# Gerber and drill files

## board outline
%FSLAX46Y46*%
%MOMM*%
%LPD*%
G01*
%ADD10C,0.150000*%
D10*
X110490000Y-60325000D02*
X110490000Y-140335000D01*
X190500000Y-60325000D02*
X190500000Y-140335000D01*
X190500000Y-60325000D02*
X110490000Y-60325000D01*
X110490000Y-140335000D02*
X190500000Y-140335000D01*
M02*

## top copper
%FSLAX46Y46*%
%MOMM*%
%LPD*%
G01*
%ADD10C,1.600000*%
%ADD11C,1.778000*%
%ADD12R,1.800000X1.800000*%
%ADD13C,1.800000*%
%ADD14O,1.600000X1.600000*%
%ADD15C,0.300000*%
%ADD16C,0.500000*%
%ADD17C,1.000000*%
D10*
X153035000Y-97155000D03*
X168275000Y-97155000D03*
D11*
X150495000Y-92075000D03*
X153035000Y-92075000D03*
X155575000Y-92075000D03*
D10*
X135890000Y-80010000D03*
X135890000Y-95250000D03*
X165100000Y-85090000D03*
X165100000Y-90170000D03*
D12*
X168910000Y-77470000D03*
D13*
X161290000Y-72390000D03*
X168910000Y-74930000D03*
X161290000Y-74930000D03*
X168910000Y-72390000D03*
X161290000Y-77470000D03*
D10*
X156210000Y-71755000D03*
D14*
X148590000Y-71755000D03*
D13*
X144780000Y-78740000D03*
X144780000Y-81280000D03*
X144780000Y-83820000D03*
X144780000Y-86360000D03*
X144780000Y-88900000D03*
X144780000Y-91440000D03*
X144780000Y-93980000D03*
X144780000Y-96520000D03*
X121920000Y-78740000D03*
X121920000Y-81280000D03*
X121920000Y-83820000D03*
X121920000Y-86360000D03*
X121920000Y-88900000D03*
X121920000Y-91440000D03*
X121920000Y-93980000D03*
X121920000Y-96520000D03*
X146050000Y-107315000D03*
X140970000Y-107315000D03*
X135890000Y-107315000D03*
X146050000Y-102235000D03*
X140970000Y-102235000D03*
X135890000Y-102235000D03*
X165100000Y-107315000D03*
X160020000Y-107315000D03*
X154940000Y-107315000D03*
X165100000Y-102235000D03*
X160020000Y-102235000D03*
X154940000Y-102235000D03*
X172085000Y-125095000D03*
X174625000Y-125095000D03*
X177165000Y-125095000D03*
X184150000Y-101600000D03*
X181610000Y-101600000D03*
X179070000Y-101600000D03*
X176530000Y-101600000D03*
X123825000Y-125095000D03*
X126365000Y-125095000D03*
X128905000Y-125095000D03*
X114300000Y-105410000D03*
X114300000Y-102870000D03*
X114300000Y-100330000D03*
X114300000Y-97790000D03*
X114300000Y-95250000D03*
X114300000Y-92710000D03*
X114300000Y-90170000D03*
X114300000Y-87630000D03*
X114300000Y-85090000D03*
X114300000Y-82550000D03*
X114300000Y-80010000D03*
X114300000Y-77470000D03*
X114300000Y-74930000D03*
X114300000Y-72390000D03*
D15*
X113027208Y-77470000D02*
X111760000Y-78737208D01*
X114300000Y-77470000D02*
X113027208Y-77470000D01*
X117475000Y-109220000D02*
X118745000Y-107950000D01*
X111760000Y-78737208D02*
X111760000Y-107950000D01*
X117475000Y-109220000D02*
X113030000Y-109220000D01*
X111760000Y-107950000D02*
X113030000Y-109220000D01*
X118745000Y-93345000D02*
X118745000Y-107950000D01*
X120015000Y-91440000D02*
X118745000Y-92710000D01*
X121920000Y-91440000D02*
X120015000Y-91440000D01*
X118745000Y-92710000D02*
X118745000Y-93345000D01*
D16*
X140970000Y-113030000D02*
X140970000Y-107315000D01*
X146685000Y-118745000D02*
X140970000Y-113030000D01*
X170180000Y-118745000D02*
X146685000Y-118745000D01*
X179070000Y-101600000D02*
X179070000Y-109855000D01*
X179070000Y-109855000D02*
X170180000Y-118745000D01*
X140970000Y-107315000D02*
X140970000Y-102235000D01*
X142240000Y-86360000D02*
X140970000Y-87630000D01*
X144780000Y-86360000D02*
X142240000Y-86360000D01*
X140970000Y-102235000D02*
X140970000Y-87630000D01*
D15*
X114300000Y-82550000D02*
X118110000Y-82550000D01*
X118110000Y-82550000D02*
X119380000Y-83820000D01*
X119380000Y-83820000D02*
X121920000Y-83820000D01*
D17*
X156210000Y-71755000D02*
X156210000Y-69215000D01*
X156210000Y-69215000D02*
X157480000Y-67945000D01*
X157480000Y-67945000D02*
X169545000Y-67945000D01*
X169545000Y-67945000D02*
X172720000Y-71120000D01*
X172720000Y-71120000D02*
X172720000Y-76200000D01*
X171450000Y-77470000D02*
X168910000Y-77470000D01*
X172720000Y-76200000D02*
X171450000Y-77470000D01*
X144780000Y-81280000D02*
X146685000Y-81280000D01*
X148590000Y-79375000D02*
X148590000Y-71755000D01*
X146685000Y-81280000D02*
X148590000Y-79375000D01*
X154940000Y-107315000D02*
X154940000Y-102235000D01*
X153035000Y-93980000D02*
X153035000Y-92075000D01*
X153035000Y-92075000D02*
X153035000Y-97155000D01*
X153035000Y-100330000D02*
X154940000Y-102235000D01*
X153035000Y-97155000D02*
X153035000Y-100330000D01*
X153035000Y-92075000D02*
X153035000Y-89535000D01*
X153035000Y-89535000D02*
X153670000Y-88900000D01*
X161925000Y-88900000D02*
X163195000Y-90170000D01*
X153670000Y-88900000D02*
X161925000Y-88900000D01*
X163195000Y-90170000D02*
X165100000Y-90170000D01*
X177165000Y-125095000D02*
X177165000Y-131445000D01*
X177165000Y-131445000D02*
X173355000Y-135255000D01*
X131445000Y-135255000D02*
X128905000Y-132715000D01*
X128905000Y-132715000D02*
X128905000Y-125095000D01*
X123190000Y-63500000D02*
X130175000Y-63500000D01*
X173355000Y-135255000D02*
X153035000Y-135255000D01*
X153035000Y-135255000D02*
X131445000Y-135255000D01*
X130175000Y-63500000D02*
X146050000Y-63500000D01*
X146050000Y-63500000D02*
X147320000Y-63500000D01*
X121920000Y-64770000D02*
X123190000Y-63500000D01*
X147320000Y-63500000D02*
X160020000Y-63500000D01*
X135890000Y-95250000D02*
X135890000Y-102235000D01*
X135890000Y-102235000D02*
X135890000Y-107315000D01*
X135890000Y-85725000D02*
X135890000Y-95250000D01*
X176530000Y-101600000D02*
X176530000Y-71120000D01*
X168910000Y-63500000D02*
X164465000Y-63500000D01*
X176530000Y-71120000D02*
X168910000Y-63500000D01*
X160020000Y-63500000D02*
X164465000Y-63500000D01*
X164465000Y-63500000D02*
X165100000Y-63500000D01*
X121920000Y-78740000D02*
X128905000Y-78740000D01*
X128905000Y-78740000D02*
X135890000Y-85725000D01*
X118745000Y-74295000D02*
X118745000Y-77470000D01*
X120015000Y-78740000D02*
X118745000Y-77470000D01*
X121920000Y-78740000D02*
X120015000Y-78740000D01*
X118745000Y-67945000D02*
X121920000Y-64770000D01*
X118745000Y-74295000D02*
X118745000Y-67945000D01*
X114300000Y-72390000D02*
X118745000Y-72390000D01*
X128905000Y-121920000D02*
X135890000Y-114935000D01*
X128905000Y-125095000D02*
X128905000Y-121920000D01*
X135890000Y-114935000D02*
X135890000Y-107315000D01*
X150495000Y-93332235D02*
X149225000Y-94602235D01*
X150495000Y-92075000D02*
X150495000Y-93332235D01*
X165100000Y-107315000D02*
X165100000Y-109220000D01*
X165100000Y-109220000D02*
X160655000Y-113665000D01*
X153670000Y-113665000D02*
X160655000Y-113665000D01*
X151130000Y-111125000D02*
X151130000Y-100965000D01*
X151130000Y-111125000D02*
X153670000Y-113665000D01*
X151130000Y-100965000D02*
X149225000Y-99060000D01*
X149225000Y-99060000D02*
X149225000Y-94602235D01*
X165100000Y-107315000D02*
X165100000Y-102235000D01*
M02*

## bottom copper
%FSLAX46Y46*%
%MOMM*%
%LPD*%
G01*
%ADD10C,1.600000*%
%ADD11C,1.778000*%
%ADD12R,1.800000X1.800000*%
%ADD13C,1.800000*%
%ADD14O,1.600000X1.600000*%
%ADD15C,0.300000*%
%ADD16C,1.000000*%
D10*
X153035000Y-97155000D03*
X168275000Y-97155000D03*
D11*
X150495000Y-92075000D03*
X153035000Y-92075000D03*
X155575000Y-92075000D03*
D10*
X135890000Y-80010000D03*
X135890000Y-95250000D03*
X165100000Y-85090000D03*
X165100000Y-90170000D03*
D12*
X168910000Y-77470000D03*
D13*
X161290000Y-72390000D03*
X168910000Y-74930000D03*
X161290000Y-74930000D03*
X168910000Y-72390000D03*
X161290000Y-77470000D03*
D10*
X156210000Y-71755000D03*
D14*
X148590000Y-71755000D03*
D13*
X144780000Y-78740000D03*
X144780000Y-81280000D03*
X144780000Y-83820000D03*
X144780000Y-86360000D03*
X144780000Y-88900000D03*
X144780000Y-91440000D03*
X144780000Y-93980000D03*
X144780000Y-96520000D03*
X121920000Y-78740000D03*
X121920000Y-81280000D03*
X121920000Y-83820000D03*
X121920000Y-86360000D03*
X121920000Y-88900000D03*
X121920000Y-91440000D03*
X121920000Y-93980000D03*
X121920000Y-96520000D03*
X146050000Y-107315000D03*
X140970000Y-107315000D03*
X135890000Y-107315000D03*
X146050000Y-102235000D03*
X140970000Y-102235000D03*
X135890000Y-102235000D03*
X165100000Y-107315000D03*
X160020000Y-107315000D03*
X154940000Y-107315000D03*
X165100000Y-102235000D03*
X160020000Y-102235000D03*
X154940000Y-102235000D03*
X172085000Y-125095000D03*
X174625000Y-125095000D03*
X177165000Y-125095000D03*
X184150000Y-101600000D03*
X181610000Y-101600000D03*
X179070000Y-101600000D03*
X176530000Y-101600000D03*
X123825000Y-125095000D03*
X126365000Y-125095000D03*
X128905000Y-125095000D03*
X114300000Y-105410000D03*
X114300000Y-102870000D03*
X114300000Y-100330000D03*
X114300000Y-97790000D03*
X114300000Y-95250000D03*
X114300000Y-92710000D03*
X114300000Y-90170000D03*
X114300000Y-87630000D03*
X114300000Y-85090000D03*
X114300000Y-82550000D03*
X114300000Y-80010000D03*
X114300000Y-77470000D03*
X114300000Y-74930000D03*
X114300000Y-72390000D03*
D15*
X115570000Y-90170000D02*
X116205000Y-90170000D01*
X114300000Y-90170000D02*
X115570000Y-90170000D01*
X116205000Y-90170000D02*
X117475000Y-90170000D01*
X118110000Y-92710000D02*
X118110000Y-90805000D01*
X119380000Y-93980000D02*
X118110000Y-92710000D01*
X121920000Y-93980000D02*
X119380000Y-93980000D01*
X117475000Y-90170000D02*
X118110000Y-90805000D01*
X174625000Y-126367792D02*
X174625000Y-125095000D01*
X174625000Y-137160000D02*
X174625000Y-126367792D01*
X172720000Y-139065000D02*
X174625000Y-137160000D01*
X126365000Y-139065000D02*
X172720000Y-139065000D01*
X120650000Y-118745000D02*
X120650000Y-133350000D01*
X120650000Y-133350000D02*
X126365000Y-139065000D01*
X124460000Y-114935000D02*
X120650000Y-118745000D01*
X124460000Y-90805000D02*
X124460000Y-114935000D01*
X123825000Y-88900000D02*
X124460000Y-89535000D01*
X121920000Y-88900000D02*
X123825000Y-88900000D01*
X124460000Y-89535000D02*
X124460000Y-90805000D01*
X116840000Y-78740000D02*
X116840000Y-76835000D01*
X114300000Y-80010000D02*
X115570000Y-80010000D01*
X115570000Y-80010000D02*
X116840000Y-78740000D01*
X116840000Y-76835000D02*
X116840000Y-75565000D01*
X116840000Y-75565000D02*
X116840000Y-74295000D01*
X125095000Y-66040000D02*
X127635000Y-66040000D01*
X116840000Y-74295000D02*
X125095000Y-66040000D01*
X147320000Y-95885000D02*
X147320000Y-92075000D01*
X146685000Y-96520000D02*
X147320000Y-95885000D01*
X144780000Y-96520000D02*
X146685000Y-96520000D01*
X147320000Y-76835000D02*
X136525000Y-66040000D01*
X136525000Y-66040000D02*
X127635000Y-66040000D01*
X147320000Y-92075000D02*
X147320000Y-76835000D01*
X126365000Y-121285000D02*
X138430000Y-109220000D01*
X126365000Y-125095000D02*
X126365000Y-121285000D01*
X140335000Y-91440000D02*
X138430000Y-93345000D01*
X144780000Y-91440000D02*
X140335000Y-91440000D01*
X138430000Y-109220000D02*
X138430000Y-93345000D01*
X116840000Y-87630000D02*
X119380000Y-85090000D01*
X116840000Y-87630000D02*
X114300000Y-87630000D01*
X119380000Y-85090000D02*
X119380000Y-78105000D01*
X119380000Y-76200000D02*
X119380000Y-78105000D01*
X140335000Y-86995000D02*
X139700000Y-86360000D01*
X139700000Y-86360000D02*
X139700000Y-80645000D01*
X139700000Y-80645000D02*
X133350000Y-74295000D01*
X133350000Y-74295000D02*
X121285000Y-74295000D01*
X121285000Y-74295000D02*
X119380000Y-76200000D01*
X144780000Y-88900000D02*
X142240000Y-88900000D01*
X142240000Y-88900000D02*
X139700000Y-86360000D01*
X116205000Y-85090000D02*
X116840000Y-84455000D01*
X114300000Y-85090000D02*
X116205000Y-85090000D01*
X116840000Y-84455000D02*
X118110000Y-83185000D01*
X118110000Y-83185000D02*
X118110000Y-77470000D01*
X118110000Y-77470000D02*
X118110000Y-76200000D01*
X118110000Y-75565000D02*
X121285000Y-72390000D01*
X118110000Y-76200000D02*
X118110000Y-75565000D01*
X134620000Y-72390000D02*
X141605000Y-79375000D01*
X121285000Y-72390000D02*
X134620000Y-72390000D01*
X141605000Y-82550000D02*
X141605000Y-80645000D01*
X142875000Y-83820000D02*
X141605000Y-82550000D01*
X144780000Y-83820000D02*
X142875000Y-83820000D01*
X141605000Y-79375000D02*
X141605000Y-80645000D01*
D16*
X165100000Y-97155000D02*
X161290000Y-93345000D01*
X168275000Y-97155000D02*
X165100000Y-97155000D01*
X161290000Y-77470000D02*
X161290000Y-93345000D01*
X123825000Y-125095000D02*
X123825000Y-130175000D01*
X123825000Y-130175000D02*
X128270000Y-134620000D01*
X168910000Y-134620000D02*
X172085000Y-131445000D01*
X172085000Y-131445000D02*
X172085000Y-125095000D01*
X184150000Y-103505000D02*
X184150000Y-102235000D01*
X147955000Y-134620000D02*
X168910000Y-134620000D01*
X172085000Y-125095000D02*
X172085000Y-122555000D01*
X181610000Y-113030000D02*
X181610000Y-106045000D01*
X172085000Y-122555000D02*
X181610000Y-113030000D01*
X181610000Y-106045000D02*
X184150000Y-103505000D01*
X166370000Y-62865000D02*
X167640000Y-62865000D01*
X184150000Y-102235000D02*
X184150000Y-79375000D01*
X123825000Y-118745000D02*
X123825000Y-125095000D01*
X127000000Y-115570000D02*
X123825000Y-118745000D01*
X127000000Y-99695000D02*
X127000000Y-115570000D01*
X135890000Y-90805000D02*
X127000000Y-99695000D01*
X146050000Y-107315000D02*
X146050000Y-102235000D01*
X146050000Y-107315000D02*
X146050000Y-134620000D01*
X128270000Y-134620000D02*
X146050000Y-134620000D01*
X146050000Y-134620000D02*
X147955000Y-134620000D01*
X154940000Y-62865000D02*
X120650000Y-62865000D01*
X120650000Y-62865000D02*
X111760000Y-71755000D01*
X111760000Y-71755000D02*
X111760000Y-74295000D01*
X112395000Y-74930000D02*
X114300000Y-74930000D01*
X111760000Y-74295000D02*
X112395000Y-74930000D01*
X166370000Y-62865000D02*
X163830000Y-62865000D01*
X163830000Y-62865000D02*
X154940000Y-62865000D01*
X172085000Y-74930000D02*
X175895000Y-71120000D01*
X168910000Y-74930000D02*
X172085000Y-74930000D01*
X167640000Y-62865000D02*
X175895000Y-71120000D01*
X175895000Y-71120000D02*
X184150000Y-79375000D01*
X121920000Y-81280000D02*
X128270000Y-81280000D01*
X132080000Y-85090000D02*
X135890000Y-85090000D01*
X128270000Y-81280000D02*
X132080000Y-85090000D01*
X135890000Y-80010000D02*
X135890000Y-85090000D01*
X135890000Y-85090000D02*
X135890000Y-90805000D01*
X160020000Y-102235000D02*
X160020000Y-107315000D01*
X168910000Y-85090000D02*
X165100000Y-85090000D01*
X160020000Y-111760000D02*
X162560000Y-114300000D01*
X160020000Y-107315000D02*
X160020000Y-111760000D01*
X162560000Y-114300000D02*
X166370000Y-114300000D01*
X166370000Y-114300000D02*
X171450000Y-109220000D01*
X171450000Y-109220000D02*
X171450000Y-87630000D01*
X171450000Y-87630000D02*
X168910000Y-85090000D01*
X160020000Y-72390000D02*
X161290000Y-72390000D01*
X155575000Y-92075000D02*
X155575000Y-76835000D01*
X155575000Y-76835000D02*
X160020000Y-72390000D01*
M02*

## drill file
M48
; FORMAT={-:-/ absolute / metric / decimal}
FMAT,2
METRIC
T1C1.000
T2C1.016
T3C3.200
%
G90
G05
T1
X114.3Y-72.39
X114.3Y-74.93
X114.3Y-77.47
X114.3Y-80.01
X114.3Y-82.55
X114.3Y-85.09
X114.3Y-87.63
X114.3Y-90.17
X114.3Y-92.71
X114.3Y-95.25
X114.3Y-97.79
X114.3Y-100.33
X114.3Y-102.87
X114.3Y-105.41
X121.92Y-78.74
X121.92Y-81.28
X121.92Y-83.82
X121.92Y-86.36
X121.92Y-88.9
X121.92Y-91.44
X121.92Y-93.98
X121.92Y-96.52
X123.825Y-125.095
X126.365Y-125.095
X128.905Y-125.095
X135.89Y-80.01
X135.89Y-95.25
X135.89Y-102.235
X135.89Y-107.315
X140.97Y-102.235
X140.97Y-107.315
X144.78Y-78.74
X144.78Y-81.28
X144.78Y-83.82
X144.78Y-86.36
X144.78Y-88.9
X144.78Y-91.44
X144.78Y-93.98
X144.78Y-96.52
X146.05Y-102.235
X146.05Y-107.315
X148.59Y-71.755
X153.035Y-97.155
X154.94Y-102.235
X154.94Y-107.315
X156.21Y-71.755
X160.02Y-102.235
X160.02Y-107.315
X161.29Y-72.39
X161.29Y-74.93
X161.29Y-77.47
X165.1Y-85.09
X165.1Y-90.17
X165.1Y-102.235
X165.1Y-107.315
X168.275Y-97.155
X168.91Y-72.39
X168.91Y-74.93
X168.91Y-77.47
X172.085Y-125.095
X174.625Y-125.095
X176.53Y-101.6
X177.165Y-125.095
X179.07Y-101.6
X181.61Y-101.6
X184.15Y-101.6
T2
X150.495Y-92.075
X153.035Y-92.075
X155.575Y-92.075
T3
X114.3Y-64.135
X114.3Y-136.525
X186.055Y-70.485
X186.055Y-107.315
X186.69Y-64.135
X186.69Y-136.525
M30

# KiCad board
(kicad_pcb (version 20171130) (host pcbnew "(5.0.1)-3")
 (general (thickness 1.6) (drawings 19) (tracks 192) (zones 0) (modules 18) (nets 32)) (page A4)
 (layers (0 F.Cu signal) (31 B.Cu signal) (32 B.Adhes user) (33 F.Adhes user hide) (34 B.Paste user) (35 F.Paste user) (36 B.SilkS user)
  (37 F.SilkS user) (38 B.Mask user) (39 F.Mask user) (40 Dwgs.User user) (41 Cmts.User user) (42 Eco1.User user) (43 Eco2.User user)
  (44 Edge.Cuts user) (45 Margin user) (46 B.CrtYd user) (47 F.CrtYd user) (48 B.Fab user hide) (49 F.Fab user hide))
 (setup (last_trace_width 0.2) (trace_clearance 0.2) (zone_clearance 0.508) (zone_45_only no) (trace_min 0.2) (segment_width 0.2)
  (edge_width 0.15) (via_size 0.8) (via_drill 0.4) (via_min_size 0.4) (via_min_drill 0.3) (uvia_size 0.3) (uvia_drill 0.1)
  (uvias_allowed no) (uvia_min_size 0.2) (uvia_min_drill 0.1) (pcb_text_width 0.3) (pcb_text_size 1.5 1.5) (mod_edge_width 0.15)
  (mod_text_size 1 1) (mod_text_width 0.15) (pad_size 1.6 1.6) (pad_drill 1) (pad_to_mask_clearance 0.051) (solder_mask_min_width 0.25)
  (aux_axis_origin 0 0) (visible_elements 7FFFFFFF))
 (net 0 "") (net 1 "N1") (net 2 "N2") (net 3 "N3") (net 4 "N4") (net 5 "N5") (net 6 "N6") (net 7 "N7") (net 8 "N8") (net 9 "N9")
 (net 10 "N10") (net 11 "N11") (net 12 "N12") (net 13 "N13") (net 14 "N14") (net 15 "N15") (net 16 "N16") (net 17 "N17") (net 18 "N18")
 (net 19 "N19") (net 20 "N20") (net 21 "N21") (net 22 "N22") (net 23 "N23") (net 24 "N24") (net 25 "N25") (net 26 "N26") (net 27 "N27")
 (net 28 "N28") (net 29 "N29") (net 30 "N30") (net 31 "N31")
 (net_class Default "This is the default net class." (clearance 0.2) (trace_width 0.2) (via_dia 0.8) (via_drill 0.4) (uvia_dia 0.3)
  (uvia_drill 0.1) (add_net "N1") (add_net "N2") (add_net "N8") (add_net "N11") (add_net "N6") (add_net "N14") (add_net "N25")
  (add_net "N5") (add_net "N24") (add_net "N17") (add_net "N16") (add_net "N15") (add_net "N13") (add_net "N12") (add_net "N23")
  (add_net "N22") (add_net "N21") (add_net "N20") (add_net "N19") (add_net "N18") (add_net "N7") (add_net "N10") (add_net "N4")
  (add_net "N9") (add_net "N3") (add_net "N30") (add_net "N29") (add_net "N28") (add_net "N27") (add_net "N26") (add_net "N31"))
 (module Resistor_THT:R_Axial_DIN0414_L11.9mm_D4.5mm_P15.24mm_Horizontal (layer F.Cu) (at 153.035 97.155)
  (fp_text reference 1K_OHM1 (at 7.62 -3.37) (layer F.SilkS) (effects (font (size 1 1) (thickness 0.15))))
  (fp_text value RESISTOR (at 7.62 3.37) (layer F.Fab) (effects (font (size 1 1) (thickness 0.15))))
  (pad 1 thru_hole circle (at 0 0) (size 1.6 1.6) (drill 1) (layers *.Cu *.Mask) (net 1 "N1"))
  (pad 2 thru_hole circle (at 15.24 0) (size 1.6 1.6) (drill 1) (layers *.Cu *.Mask) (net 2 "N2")))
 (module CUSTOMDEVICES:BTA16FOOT (layer F.Cu) (at 153.035 86.995)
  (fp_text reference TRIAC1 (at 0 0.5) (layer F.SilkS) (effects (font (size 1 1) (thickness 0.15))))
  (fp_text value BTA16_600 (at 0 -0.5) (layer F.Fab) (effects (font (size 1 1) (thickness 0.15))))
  (pad 1 thru_hole circle (at -2.54 5.08) (size 1.778 1.778) (drill 1.016) (layers *.Cu *.Mask) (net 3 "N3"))
  (pad 2 thru_hole circle (at 0 5.08) (size 1.778 1.778) (drill 1.016) (layers *.Cu *.Mask) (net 1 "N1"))
  (pad 3 thru_hole circle (at 2.54 5.08) (size 1.778 1.778) (drill 1.016) (layers *.Cu *.Mask) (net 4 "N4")))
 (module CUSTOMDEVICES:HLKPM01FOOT (layer B.Cu) (at 150.495 87.63 180)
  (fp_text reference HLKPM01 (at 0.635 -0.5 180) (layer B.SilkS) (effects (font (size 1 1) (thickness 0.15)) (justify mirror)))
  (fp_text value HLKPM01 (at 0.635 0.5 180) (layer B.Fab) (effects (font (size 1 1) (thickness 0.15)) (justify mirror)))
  (pad 3 thru_hole circle (at 14.605 7.62 180) (size 1.6 1.6) (drill 1) (layers *.Cu *.Mask) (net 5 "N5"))
  (pad 4 thru_hole circle (at 14.605 -7.62 180) (size 1.6 1.6) (drill 1) (layers *.Cu *.Mask) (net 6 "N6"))
  (pad 1 thru_hole circle (at -14.605 2.54 180) (size 1.6 1.6) (drill 1) (layers *.Cu *.Mask) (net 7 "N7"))
  (pad 2 thru_hole circle (at -14.605 -2.54 180) (size 1.6 1.6) (drill 1) (layers *.Cu *.Mask) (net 1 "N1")))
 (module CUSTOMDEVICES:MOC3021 (layer F.Cu) (at 168.91 77.47 180)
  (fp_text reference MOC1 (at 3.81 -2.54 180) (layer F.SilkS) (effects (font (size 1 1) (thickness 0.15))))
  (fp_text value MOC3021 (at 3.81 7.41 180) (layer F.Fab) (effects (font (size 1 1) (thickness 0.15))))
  (pad 1 thru_hole rect (at 0 0 180) (size 1.8 1.8) (drill 1) (layers *.Cu *.Mask) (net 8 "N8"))
  (pad 4 thru_hole circle (at 7.62 5.08 180) (size 1.8 1.8) (drill 1) (layers *.Cu *.Mask) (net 4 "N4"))
  (pad 2 thru_hole circle (at 0 2.54 180) (size 1.8 1.8) (drill 1) (layers *.Cu *.Mask) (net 5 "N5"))
  (pad 5 thru_hole circle (at 7.62 2.54 180) (size 1.8 1.8) (drill 1) (layers *.Cu *.Mask) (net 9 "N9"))
  (pad 3 thru_hole circle (at 0 5.08 180) (size 1.8 1.8) (drill 1) (layers *.Cu *.Mask) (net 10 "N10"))
  (pad 6 thru_hole circle (at 7.62 0 180) (size 1.8 1.8) (drill 1) (layers *.Cu *.Mask) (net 2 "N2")))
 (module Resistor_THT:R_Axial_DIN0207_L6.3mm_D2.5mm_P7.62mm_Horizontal (layer F.Cu) (at 156.21 71.755 180)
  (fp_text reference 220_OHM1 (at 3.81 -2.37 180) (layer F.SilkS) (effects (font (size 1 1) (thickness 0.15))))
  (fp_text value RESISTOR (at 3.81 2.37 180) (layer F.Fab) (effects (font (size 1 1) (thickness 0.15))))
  (pad 1 thru_hole circle (at 0 0 180) (size 1.6 1.6) (drill 1) (layers *.Cu *.Mask) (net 8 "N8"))
  (pad 2 thru_hole oval (at 7.62 0 180) (size 1.6 1.6) (drill 1) (layers *.Cu *.Mask) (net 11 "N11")))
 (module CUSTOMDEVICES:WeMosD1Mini (layer F.Cu) (at 133.35 86.36 180)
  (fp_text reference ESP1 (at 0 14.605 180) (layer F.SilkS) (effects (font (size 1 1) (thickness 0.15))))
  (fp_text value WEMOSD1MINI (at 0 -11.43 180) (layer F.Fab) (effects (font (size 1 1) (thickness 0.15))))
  (pad 16 thru_hole circle (at -11.43 7.62 180) (size 1.8 1.8) (drill 1) (layers *.Cu *.Mask) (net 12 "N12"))
  (pad 15 thru_hole circle (at -11.43 5.08 180) (size 1.8 1.8) (drill 1) (layers *.Cu *.Mask) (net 11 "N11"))
  (pad 14 thru_hole circle (at -11.43 2.54 180) (size 1.8 1.8) (drill 1) (layers *.Cu *.Mask) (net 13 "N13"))
  (pad 13 thru_hole circle (at -11.43 0 180) (size 1.8 1.8) (drill 1) (layers *.Cu *.Mask) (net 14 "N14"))
  (pad 12 thru_hole circle (at -11.43 -2.54 180) (size 1.8 1.8) (drill 1) (layers *.Cu *.Mask) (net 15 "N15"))
  (pad 11 thru_hole circle (at -11.43 -5.08 180) (size 1.8 1.8) (drill 1) (layers *.Cu *.Mask) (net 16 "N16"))
  (pad 10 thru_hole circle (at -11.43 -7.62 180) (size 1.8 1.8) (drill 1) (layers *.Cu *.Mask) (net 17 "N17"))
  (pad 9 thru_hole circle (at -11.43 -10.16 180) (size 1.8 1.8) (drill 1) (layers *.Cu *.Mask) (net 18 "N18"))
  (pad 8 thru_hole circle (at 11.43 7.62 180) (size 1.8 1.8) (drill 1) (layers *.Cu *.Mask) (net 6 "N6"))
  (pad 7 thru_hole circle (at 11.43 5.08 180) (size 1.8 1.8) (drill 1) (layers *.Cu *.Mask) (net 5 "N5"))
  (pad 6 thru_hole circle (at 11.43 2.54 180) (size 1.8 1.8) (drill 1) (layers *.Cu *.Mask) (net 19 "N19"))
  (pad 5 thru_hole circle (at 11.43 0 180) (size 1.8 1.8) (drill 1) (layers *.Cu *.Mask) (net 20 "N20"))
  (pad 4 thru_hole circle (at 11.43 -2.54 180) (size 1.8 1.8) (drill 1) (layers *.Cu *.Mask) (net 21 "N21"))
  (pad 3 thru_hole circle (at 11.43 -5.08 180) (size 1.8 1.8) (drill 1) (layers *.Cu *.Mask) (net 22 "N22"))
  (pad 2 thru_hole circle (at 11.43 -7.62 180) (size 1.8 1.8) (drill 1) (layers *.Cu *.Mask) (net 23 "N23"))
  (pad 1 thru_hole circle (at 11.43 -10.16 180) (size 1.8 1.8) (drill 1) (layers *.Cu *.Mask) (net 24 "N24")))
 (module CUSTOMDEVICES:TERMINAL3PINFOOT (layer B.Cu) (at 140.97 104.775)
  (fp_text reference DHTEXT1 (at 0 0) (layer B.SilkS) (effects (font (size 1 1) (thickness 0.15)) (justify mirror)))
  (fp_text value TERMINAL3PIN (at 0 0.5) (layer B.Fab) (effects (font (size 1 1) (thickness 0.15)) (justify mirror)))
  (pad 3 thru_hole circle (at 5.08 2.54) (size 1.8 1.8) (drill 1) (layers *.Cu *.Mask) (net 5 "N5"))
  (pad 2 thru_hole circle (at 0 2.54) (size 1.8 1.8) (drill 1) (layers *.Cu *.Mask) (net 14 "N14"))
  (pad 1 thru_hole circle (at -5.08 2.54) (size 1.8 1.8) (drill 1) (layers *.Cu *.Mask) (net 6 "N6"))
  (pad 3 thru_hole circle (at 5.08 -2.54) (size 1.8 1.8) (drill 1) (layers *.Cu *.Mask) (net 5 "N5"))
  (pad 2 thru_hole circle (at 0 -2.54) (size 1.8 1.8) (drill 1) (layers *.Cu *.Mask) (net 14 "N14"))
  (pad 1 thru_hole circle (at -5.08 -2.54) (size 1.8 1.8) (drill 1) (layers *.Cu *.Mask) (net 6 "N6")))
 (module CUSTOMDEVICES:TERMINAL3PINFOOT (layer B.Cu) (at 160.02 104.775)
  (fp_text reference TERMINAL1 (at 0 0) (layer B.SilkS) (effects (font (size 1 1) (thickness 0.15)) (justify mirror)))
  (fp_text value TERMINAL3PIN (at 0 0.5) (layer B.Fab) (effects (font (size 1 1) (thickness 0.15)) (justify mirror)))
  (pad 3 thru_hole circle (at 5.08 2.54) (size 1.8 1.8) (drill 1) (layers *.Cu *.Mask) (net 3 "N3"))
  (pad 2 thru_hole circle (at 0 2.54) (size 1.8 1.8) (drill 1) (layers *.Cu *.Mask) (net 7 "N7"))
  (pad 1 thru_hole circle (at -5.08 2.54) (size 1.8 1.8) (drill 1) (layers *.Cu *.Mask) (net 1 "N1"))
  (pad 3 thru_hole circle (at 5.08 -2.54) (size 1.8 1.8) (drill 1) (layers *.Cu *.Mask) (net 3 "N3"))
  (pad 2 thru_hole circle (at 0 -2.54) (size 1.8 1.8) (drill 1) (layers *.Cu *.Mask) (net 7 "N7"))
  (pad 1 thru_hole circle (at -5.08 -2.54) (size 1.8 1.8) (drill 1) (layers *.Cu *.Mask) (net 1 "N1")))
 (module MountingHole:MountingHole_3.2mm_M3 (layer F.Cu) (at 186.055 107.315)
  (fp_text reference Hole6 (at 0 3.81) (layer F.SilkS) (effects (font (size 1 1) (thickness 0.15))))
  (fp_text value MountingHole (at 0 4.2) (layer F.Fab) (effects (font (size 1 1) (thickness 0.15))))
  (pad 1 np_thru_hole circle (at 0 0) (size 3.2 3.2) (drill 3.2) (layers *.Cu *.Mask)))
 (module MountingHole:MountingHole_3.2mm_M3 (layer F.Cu) (at 186.055 70.485)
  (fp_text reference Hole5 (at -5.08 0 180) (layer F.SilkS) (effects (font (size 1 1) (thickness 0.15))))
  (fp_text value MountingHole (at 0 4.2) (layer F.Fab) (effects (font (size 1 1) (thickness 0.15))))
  (pad 1 np_thru_hole circle (at 0 0) (size 3.2 3.2) (drill 3.2) (layers *.Cu *.Mask)))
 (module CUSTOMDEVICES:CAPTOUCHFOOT (layer F.Cu) (at 174.625 130.175 180)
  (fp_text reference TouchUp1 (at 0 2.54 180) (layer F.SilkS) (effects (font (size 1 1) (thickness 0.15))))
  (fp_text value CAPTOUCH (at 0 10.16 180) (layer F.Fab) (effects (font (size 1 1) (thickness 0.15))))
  (pad 3 thru_hole circle (at 2.54 5.08 180) (size 1.8 1.8) (drill 1) (layers *.Cu *.Mask) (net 5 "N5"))
  (pad 2 thru_hole circle (at 0 5.08 180) (size 1.8 1.8) (drill 1) (layers *.Cu *.Mask) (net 21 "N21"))
  (pad 1 thru_hole circle (at -2.54 5.08 180) (size 1.8 1.8) (drill 1) (layers *.Cu *.Mask) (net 6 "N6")))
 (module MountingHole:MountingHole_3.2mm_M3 (layer F.Cu) (at 186.69 136.525)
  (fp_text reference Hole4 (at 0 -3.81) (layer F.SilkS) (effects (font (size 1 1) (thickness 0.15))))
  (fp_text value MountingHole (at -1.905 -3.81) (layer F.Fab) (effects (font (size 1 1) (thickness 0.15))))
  (pad 1 np_thru_hole circle (at 0 0) (size 3.2 3.2) (drill 3.2) (layers *.Cu *.Mask)))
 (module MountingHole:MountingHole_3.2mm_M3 (layer F.Cu) (at 114.3 136.525)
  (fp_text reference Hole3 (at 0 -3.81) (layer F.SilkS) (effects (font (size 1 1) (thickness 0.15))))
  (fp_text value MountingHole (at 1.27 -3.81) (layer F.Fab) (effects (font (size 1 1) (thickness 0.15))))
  (pad 1 np_thru_hole circle (at 0 0) (size 3.2 3.2) (drill 3.2) (layers *.Cu *.Mask)))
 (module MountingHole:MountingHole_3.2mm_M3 (layer F.Cu) (at 186.69 64.135)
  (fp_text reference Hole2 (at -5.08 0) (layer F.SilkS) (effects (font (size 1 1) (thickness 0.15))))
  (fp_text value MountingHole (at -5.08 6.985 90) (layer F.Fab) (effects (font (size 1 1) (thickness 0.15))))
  (pad 1 np_thru_hole circle (at 0 0) (size 3.2 3.2) (drill 3.2) (layers *.Cu *.Mask)))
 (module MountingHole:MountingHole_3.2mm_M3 (layer F.Cu) (at 114.3 64.135)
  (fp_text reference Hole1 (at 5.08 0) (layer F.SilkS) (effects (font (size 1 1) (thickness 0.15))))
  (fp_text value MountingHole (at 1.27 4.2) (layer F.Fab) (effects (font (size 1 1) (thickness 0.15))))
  (pad 1 np_thru_hole circle (at 0 0) (size 3.2 3.2) (drill 3.2) (layers *.Cu *.Mask)))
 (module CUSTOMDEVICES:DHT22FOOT (layer F.Cu) (at 181.61 88.9)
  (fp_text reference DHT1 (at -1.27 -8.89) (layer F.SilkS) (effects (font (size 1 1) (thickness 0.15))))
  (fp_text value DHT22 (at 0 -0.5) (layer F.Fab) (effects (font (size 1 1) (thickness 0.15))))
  (pad 4 thru_hole circle (at 2.54 12.7) (size 1.8 1.8) (drill 1) (layers *.Cu *.Mask) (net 5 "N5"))
  (pad 3 thru_hole circle (at 0 12.7) (size 1.8 1.8) (drill 1) (layers *.Cu *.Mask) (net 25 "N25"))
  (pad 2 thru_hole circle (at -2.54 12.7) (size 1.8 1.8) (drill 1) (layers *.Cu *.Mask) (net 14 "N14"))
  (pad 1 thru_hole circle (at -5.08 12.7) (size 1.8 1.8) (drill 1) (layers *.Cu *.Mask) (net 6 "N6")))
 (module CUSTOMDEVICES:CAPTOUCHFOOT (layer F.Cu) (at 126.365 130.175 180)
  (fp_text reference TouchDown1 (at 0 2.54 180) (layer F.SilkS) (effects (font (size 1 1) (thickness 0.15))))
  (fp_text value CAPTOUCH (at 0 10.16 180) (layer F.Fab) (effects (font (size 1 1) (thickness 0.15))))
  (pad 3 thru_hole circle (at 2.54 5.08 180) (size 1.8 1.8) (drill 1) (layers *.Cu *.Mask) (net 5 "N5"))
  (pad 2 thru_hole circle (at 0 5.08 180) (size 1.8 1.8) (drill 1) (layers *.Cu *.Mask) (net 16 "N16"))
  (pad 1 thru_hole circle (at -2.54 5.08 180) (size 1.8 1.8) (drill 1) (layers *.Cu *.Mask) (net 6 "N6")))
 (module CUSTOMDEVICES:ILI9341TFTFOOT (layer F.Cu) (at 116.84 90.17 180)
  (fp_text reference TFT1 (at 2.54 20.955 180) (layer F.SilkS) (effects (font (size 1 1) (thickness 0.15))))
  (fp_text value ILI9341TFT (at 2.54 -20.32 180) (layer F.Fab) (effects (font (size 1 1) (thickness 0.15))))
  (pad 14 thru_hole circle (at 2.54 -15.24 180) (size 1.8 1.8) (drill 1) (layers *.Cu *.Mask) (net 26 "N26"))
  (pad 13 thru_hole circle (at 2.54 -12.7 180) (size 1.8 1.8) (drill 1) (layers *.Cu *.Mask) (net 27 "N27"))
  (pad 12 thru_hole circle (at 2.54 -10.16 180) (size 1.8 1.8) (drill 1) (layers *.Cu *.Mask) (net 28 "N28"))
  (pad 11 thru_hole circle (at 2.54 -7.62 180) (size 1.8 1.8) (drill 1) (layers *.Cu *.Mask) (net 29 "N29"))
  (pad 10 thru_hole circle (at 2.54 -5.08 180) (size 1.8 1.8) (drill 1) (layers *.Cu *.Mask) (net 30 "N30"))
  (pad 9 thru_hole circle (at 2.54 -2.54 180) (size 1.8 1.8) (drill 1) (layers *.Cu *.Mask) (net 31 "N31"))
  (pad 8 thru_hole circle (at 2.54 0 180) (size 1.8 1.8) (drill 1) (layers *.Cu *.Mask) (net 23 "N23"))
  (pad 7 thru_hole circle (at 2.54 2.54 180) (size 1.8 1.8) (drill 1) (layers *.Cu *.Mask) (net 15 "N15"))
  (pad 6 thru_hole circle (at 2.54 5.08 180) (size 1.8 1.8) (drill 1) (layers *.Cu *.Mask) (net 13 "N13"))
  (pad 5 thru_hole circle (at 2.54 7.62 180) (size 1.8 1.8) (drill 1) (layers *.Cu *.Mask) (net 19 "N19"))
  (pad 4 thru_hole circle (at 2.54 10.16 180) (size 1.8 1.8) (drill 1) (layers *.Cu *.Mask) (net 18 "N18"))
  (pad 3 thru_hole circle (at 2.54 12.7 180) (size 1.8 1.8) (drill 1) (layers *.Cu *.Mask) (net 22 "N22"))
  (pad 2 thru_hole circle (at 2.54 15.24 180) (size 1.8 1.8) (drill 1) (layers *.Cu *.Mask) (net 5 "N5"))
  (pad 1 thru_hole circle (at 2.54 17.78 180) (size 1.8 1.8) (drill 1) (layers *.Cu *.Mask) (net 6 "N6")))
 (gr_line (start 110.49 60.325) (end 110.49 140.335) (layer Edge.Cuts) (width 0.15))
 (gr_line (start 190.5 60.325) (end 190.5 140.335) (layer Edge.Cuts) (width 0.15))
 (gr_line (start 190.5 60.325) (end 110.49 60.325) (layer Edge.Cuts) (width 0.15))
 (gr_line (start 110.49 140.335) (end 190.5 140.335) (layer Edge.Cuts) (width 0.15))
 (segment (start 115.57 90.17) (end 116.205 90.17) (width 0.3) (layer B.Cu) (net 23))
 (segment (start 114.3 90.17) (end 115.57 90.17) (width 0.3) (layer B.Cu) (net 23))
 (segment (start 116.205 90.17) (end 117.475 90.17) (width 0.3) (layer B.Cu) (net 23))
 (segment (start 118.11 92.71) (end 118.11 90.805) (width 0.3) (layer B.Cu) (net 23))
 (segment (start 119.38 93.98) (end 118.11 92.71) (width 0.3) (layer B.Cu) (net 23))
 (segment (start 121.92 93.98) (end 119.38 93.98) (width 0.3) (layer B.Cu) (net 23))
 (segment (start 117.475 90.17) (end 118.11 90.805) (width 0.3) (layer B.Cu) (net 23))
 (segment (start 113.027208 77.47) (end 111.76 78.737208) (width 0.3) (layer F.Cu) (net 22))
 (segment (start 114.3 77.47) (end 113.027208 77.47) (width 0.3) (layer F.Cu) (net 22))
 (segment (start 117.475 109.22) (end 118.745 107.95) (width 0.3) (layer F.Cu) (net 22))
 (segment (start 111.76 78.737208) (end 111.76 107.95) (width 0.3) (layer F.Cu) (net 22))
 (segment (start 117.475 109.22) (end 113.03 109.22) (width 0.3) (layer F.Cu) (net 22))
 (segment (start 111.76 107.95) (end 113.03 109.22) (width 0.3) (layer F.Cu) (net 22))
 (segment (start 118.745 93.345) (end 118.745 107.95) (width 0.3) (layer F.Cu) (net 22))
 (segment (start 120.015 91.44) (end 118.745 92.71) (width 0.3) (layer F.Cu) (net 22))
 (segment (start 121.92 91.44) (end 120.015 91.44) (width 0.3) (layer F.Cu) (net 22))
 (segment (start 118.745 92.71) (end 118.745 93.345) (width 0.3) (layer F.Cu) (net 22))
 (segment (start 174.625 126.367792) (end 174.625 125.095) (width 0.3) (layer B.Cu) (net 21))
 (segment (start 174.625 137.16) (end 174.625 126.367792) (width 0.3) (layer B.Cu) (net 21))
 (segment (start 172.72 139.065) (end 174.625 137.16) (width 0.3) (layer B.Cu) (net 21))
 (segment (start 126.365 139.065) (end 172.72 139.065) (width 0.3) (layer B.Cu) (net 21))
 (segment (start 120.65 118.745) (end 120.65 133.35) (width 0.3) (layer B.Cu) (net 21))
 (segment (start 120.65 133.35) (end 126.365 139.065) (width 0.3) (layer B.Cu) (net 21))
 (segment (start 124.46 114.935) (end 120.65 118.745) (width 0.3) (layer B.Cu) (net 21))
 (segment (start 124.46 90.805) (end 124.46 114.935) (width 0.3) (layer B.Cu) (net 21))
 (segment (start 123.825 88.9) (end 124.46 89.535) (width 0.3) (layer B.Cu) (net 21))
 (segment (start 121.92 88.9) (end 123.825 88.9) (width 0.3) (layer B.Cu) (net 21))
 (segment (start 124.46 89.535) (end 124.46 90.805) (width 0.3) (layer B.Cu) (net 21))
 (segment (start 140.97 113.03) (end 140.97 107.315) (width 0.5) (layer F.Cu) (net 14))
 (segment (start 146.685 118.745) (end 140.97 113.03) (width 0.5) (layer F.Cu) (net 14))
 (segment (start 170.18 118.745) (end 146.685 118.745) (width 0.5) (layer F.Cu) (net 14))
 (segment (start 179.07 101.6) (end 179.07 109.855) (width 0.5) (layer F.Cu) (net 14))
 (segment (start 179.07 109.855) (end 170.18 118.745) (width 0.5) (layer F.Cu) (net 14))
 (segment (start 140.97 107.315) (end 140.97 102.235) (width 0.5) (layer F.Cu) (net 14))
 (segment (start 142.24 86.36) (end 140.97 87.63) (width 0.5) (layer F.Cu) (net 14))
 (segment (start 144.78 86.36) (end 142.24 86.36) (width 0.5) (layer F.Cu) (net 14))
 (segment (start 140.97 102.235) (end 140.97 87.63) (width 0.5) (layer F.Cu) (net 14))
 (segment (start 114.3 82.55) (end 118.11 82.55) (width 0.3) (layer F.Cu) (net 19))
 (segment (start 118.11 82.55) (end 119.38 83.82) (width 0.3) (layer F.Cu) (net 19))
 (segment (start 119.38 83.82) (end 121.92 83.82) (width 0.3) (layer F.Cu) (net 19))
 (segment (start 116.84 78.74) (end 116.84 76.835) (width 0.3) (layer B.Cu) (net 18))
 (segment (start 114.3 80.01) (end 115.57 80.01) (width 0.3) (layer B.Cu) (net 18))
 (segment (start 115.57 80.01) (end 116.84 78.74) (width 0.3) (layer B.Cu) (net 18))
 (segment (start 116.84 76.835) (end 116.84 75.565) (width 0.3) (layer B.Cu) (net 18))
 (segment (start 116.84 75.565) (end 116.84 74.295) (width 0.3) (layer B.Cu) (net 18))
 (segment (start 125.095 66.04) (end 127.635 66.04) (width 0.3) (layer B.Cu) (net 18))
 (segment (start 116.84 74.295) (end 125.095 66.04) (width 0.3) (layer B.Cu) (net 18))
 (segment (start 147.32 95.885) (end 147.32 92.075) (width 0.3) (layer B.Cu) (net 18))
 (segment (start 146.685 96.52) (end 147.32 95.885) (width 0.3) (layer B.Cu) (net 18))
 (segment (start 144.78 96.52) (end 146.685 96.52) (width 0.3) (layer B.Cu) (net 18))
 (segment (start 147.32 76.835) (end 136.525 66.04) (width 0.3) (layer B.Cu) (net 18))
 (segment (start 136.525 66.04) (end 127.635 66.04) (width 0.3) (layer B.Cu) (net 18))
 (segment (start 147.32 92.075) (end 147.32 76.835) (width 0.3) (layer B.Cu) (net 18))
 (segment (start 126.365 121.285) (end 138.43 109.22) (width 0.3) (layer B.Cu) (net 16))
 (segment (start 126.365 125.095) (end 126.365 121.285) (width 0.3) (layer B.Cu) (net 16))
 (segment (start 140.335 91.44) (end 138.43 93.345) (width 0.3) (layer B.Cu) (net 16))
 (segment (start 144.78 91.44) (end 140.335 91.44) (width 0.3) (layer B.Cu) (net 16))
 (segment (start 138.43 109.22) (end 138.43 93.345) (width 0.3) (layer B.Cu) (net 16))
 (segment (start 116.84 87.63) (end 119.38 85.09) (width 0.3) (layer B.Cu) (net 15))
 (segment (start 116.84 87.63) (end 114.3 87.63) (width 0.3) (layer B.Cu) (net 15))
 (segment (start 119.38 85.09) (end 119.38 78.105) (width 0.3) (layer B.Cu) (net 15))
 (segment (start 119.38 76.2) (end 119.38 78.105) (width 0.3) (layer B.Cu) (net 15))
 (segment (start 140.335 86.995) (end 139.7 86.36) (width 0.3) (layer B.Cu) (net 15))
 (segment (start 139.7 86.36) (end 139.7 80.645) (width 0.3) (layer B.Cu) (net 15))
 (segment (start 139.7 80.645) (end 133.35 74.295) (width 0.3) (layer B.Cu) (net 15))
 (segment (start 133.35 74.295) (end 121.285 74.295) (width 0.3) (layer B.Cu) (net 15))
 (segment (start 121.285 74.295) (end 119.38 76.2) (width 0.3) (layer B.Cu) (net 15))
 (segment (start 144.78 88.9) (end 142.24 88.9) (width 0.3) (layer B.Cu) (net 15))
 (segment (start 142.24 88.9) (end 139.7 86.36) (width 0.3) (layer B.Cu) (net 15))
 (segment (start 116.205 85.09) (end 116.84 84.455) (width 0.3) (layer B.Cu) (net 13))
 (segment (start 114.3 85.09) (end 116.205 85.09) (width 0.3) (layer B.Cu) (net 13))
 (segment (start 116.84 84.455) (end 118.11 83.185) (width 0.3) (layer B.Cu) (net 13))
 (segment (start 118.11 83.185) (end 118.11 77.47) (width 0.3) (layer B.Cu) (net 13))
 (segment (start 118.11 77.47) (end 118.11 76.2) (width 0.3) (layer B.Cu) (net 13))
 (segment (start 118.11 75.565) (end 121.285 72.39) (width 0.3) (layer B.Cu) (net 13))
 (segment (start 118.11 76.2) (end 118.11 75.565) (width 0.3) (layer B.Cu) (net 13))
 (segment (start 134.62 72.39) (end 141.605 79.375) (width 0.3) (layer B.Cu) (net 13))
 (segment (start 121.285 72.39) (end 134.62 72.39) (width 0.3) (layer B.Cu) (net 13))
 (segment (start 141.605 82.55) (end 141.605 80.645) (width 0.3) (layer B.Cu) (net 13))
 (segment (start 142.875 83.82) (end 141.605 82.55) (width 0.3) (layer B.Cu) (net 13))
 (segment (start 144.78 83.82) (end 142.875 83.82) (width 0.3) (layer B.Cu) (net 13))
 (segment (start 141.605 79.375) (end 141.605 80.645) (width 0.3) (layer B.Cu) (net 13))
 (segment (start 156.21 71.755) (end 156.21 69.215) (width 1) (layer F.Cu) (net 8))
 (segment (start 156.21 69.215) (end 157.48 67.945) (width 1) (layer F.Cu) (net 8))
 (segment (start 157.48 67.945) (end 169.545 67.945) (width 1) (layer F.Cu) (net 8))
 (segment (start 169.545 67.945) (end 172.72 71.12) (width 1) (layer F.Cu) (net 8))
 (segment (start 172.72 71.12) (end 172.72 76.2) (width 1) (layer F.Cu) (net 8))
 (segment (start 171.45 77.47) (end 168.91 77.47) (width 1) (layer F.Cu) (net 8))
 (segment (start 172.72 76.2) (end 171.45 77.47) (width 1) (layer F.Cu) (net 8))
 (segment (start 144.78 81.28) (end 146.685 81.28) (width 1) (layer F.Cu) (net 11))
 (segment (start 148.59 79.375) (end 148.59 71.755) (width 1) (layer F.Cu) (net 11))
 (segment (start 146.685 81.28) (end 148.59 79.375) (width 1) (layer F.Cu) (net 11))
 (segment (start 165.1 97.155) (end 161.29 93.345) (width 1) (layer B.Cu) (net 2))
 (segment (start 168.275 97.155) (end 165.1 97.155) (width 1) (layer B.Cu) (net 2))
 (segment (start 161.29 77.47) (end 161.29 93.345) (width 1) (layer B.Cu) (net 2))
 (segment (start 154.94 107.315) (end 154.94 102.235) (width 1) (layer F.Cu) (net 1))
 (segment (start 153.035 93.98) (end 153.035 92.075) (width 1) (layer F.Cu) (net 1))
 (segment (start 153.035 92.075) (end 153.035 97.155) (width 1) (layer F.Cu) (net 1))
 (segment (start 153.035 100.33) (end 154.94 102.235) (width 1) (layer F.Cu) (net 1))
 (segment (start 153.035 97.155) (end 153.035 100.33) (width 1) (layer F.Cu) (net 1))
 (segment (start 153.035 92.075) (end 153.035 89.535) (width 1) (layer F.Cu) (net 1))
 (segment (start 153.035 89.535) (end 153.67 88.9) (width 1) (layer F.Cu) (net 1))
 (segment (start 161.925 88.9) (end 163.195 90.17) (width 1) (layer F.Cu) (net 1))
 (segment (start 153.67 88.9) (end 161.925 88.9) (width 1) (layer F.Cu) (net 1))
 (segment (start 163.195 90.17) (end 165.1 90.17) (width 1) (layer F.Cu) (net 1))
 (segment (start 177.165 125.095) (end 177.165 131.445) (width 1) (layer F.Cu) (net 6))
 (segment (start 177.165 131.445) (end 173.355 135.255) (width 1) (layer F.Cu) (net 6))
 (segment (start 131.445 135.255) (end 128.905 132.715) (width 1) (layer F.Cu) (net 6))
 (segment (start 128.905 132.715) (end 128.905 125.095) (width 1) (layer F.Cu) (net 6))
 (segment (start 123.19 63.5) (end 130.175 63.5) (width 1) (layer F.Cu) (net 6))
 (segment (start 173.355 135.255) (end 153.035 135.255) (width 1) (layer F.Cu) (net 6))
 (segment (start 153.035 135.255) (end 131.445 135.255) (width 1) (layer F.Cu) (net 6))
 (segment (start 130.175 63.5) (end 146.05 63.5) (width 1) (layer F.Cu) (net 6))
 (segment (start 146.05 63.5) (end 147.32 63.5) (width 1) (layer F.Cu) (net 6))
 (segment (start 121.92 64.77) (end 123.19 63.5) (width 1) (layer F.Cu) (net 6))
 (segment (start 147.32 63.5) (end 160.02 63.5) (width 1) (layer F.Cu) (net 6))
 (segment (start 135.89 95.25) (end 135.89 102.235) (width 1) (layer F.Cu) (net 6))
 (segment (start 135.89 102.235) (end 135.89 107.315) (width 1) (layer F.Cu) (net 6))
 (segment (start 135.89 85.725) (end 135.89 95.25) (width 1) (layer F.Cu) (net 6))
 (segment (start 176.53 101.6) (end 176.53 71.12) (width 1) (layer F.Cu) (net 6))
 (segment (start 168.91 63.5) (end 164.465 63.5) (width 1) (layer F.Cu) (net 6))
 (segment (start 176.53 71.12) (end 168.91 63.5) (width 1) (layer F.Cu) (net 6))
 (segment (start 160.02 63.5) (end 164.465 63.5) (width 1) (layer F.Cu) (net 6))
 (segment (start 164.465 63.5) (end 165.1 63.5) (width 1) (layer F.Cu) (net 6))
 (segment (start 121.92 78.74) (end 128.905 78.74) (width 1) (layer F.Cu) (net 6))
 (segment (start 128.905 78.74) (end 135.89 85.725) (width 1) (layer F.Cu) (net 6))
 (segment (start 118.745 74.295) (end 118.745 77.47) (width 1) (layer F.Cu) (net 6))
 (segment (start 120.015 78.74) (end 118.745 77.47) (width 1) (layer F.Cu) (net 6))
 (segment (start 121.92 78.74) (end 120.015 78.74) (width 1) (layer F.Cu) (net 6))
 (segment (start 118.745 67.945) (end 121.92 64.77) (width 1) (layer F.Cu) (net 6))
 (segment (start 118.745 74.295) (end 118.745 67.945) (width 1) (layer F.Cu) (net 6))
 (segment (start 114.3 72.39) (end 118.745 72.39) (width 1) (layer F.Cu) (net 6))
 (segment (start 128.905 121.92) (end 135.89 114.935) (width 1) (layer F.Cu) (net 6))
 (segment (start 128.905 125.095) (end 128.905 121.92) (width 1) (layer F.Cu) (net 6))
 (segment (start 135.89 114.935) (end 135.89 107.315) (width 1) (layer F.Cu) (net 6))
 (segment (start 123.825 125.095) (end 123.825 130.175) (width 1) (layer B.Cu) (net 5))
 (segment (start 123.825 130.175) (end 128.27 134.62) (width 1) (layer B.Cu) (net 5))
 (segment (start 168.91 134.62) (end 172.085 131.445) (width 1) (layer B.Cu) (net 5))
 (segment (start 172.085 131.445) (end 172.085 125.095) (width 1) (layer B.Cu) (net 5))
 (segment (start 184.15 103.505) (end 184.15 102.235) (width 1) (layer B.Cu) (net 5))
 (segment (start 147.955 134.62) (end 168.91 134.62) (width 1) (layer B.Cu) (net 5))
 (segment (start 172.085 125.095) (end 172.085 122.555) (width 1) (layer B.Cu) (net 5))
 (segment (start 181.61 113.03) (end 181.61 106.045) (width 1) (layer B.Cu) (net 5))
 (segment (start 172.085 122.555) (end 181.61 113.03) (width 1) (layer B.Cu) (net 5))
 (segment (start 181.61 106.045) (end 184.15 103.505) (width 1) (layer B.Cu) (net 5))
 (segment (start 166.37 62.865) (end 167.64 62.865) (width 1) (layer B.Cu) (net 5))
 (segment (start 184.15 102.235) (end 184.15 79.375) (width 1) (layer B.Cu) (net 5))
 (segment (start 123.825 118.745) (end 123.825 125.095) (width 1) (layer B.Cu) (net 5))
 (segment (start 127 115.57) (end 123.825 118.745) (width 1) (layer B.Cu) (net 5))
 (segment (start 127 99.695) (end 127 115.57) (width 1) (layer B.Cu) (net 5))
 (segment (start 135.89 90.805) (end 127 99.695) (width 1) (layer B.Cu) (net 5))
 (segment (start 146.05 107.315) (end 146.05 102.235) (width 1) (layer B.Cu) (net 5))
 (segment (start 146.05 107.315) (end 146.05 134.62) (width 1) (layer B.Cu) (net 5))
 (segment (start 128.27 134.62) (end 146.05 134.62) (width 1) (layer B.Cu) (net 5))
 (segment (start 146.05 134.62) (end 147.955 134.62) (width 1) (layer B.Cu) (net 5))
 (segment (start 154.94 62.865) (end 120.65 62.865) (width 1) (layer B.Cu) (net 5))
 (segment (start 120.65 62.865) (end 111.76 71.755) (width 1) (layer B.Cu) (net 5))
 (segment (start 111.76 71.755) (end 111.76 74.295) (width 1) (layer B.Cu) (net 5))
 (segment (start 112.395 74.93) (end 114.3 74.93) (width 1) (layer B.Cu) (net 5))
 (segment (start 111.76 74.295) (end 112.395 74.93) (width 1) (layer B.Cu) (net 5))
 (segment (start 166.37 62.865) (end 163.83 62.865) (width 1) (layer B.Cu) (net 5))
 (segment (start 163.83 62.865) (end 154.94 62.865) (width 1) (layer B.Cu) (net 5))
 (segment (start 172.085 74.93) (end 175.895 71.12) (width 1) (layer B.Cu) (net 5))
 (segment (start 168.91 74.93) (end 172.085 74.93) (width 1) (layer B.Cu) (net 5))
 (segment (start 167.64 62.865) (end 175.895 71.12) (width 1) (layer B.Cu) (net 5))
 (segment (start 175.895 71.12) (end 184.15 79.375) (width 1) (layer B.Cu) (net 5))
 (segment (start 121.92 81.28) (end 128.27 81.28) (width 1) (layer B.Cu) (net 5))
 (segment (start 132.08 85.09) (end 135.89 85.09) (width 1) (layer B.Cu) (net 5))
 (segment (start 128.27 81.28) (end 132.08 85.09) (width 1) (layer B.Cu) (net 5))
 (segment (start 135.89 80.01) (end 135.89 85.09) (width 1) (layer B.Cu) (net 5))
 (segment (start 135.89 85.09) (end 135.89 90.805) (width 1) (layer B.Cu) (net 5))
 (segment (start 150.495 93.332235) (end 149.225 94.602235) (width 1) (layer F.Cu) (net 3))
 (segment (start 150.495 92.075) (end 150.495 93.332235) (width 1) (layer F.Cu) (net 3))
 (segment (start 165.1 107.315) (end 165.1 109.22) (width 1) (layer F.Cu) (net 3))
 (segment (start 165.1 109.22) (end 160.655 113.665) (width 1) (layer F.Cu) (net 3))
 (segment (start 153.67 113.665) (end 160.655 113.665) (width 1) (layer F.Cu) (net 3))
 (segment (start 151.13 111.125) (end 151.13 100.965) (width 1) (layer F.Cu) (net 3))
 (segment (start 151.13 111.125) (end 153.67 113.665) (width 1) (layer F.Cu) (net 3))
 (segment (start 151.13 100.965) (end 149.225 99.06) (width 1) (layer F.Cu) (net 3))
 (segment (start 149.225 99.06) (end 149.225 94.602235) (width 1) (layer F.Cu) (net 3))
 (segment (start 165.1 107.315) (end 165.1 102.235) (width 1) (layer F.Cu) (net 3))
 (segment (start 160.02 102.235) (end 160.02 107.315) (width 1) (layer B.Cu) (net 7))
 (segment (start 168.91 85.09) (end 165.1 85.09) (width 1) (layer B.Cu) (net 7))
 (segment (start 160.02 111.76) (end 162.56 114.3) (width 1) (layer B.Cu) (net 7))
 (segment (start 160.02 107.315) (end 160.02 111.76) (width 1) (layer B.Cu) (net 7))
 (segment (start 162.56 114.3) (end 166.37 114.3) (width 1) (layer B.Cu) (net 7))
 (segment (start 166.37 114.3) (end 171.45 109.22) (width 1) (layer B.Cu) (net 7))
 (segment (start 171.45 109.22) (end 171.45 87.63) (width 1) (layer B.Cu) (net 7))
 (segment (start 171.45 87.63) (end 168.91 85.09) (width 1) (layer B.Cu) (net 7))
 (segment (start 160.02 72.39) (end 161.29 72.39) (width 1) (layer B.Cu) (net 4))
 (segment (start 155.575 92.075) (end 155.575 76.835) (width 1) (layer B.Cu) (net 4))
 (segment (start 155.575 76.835) (end 160.02 72.39) (width 1) (layer B.Cu) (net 4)))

